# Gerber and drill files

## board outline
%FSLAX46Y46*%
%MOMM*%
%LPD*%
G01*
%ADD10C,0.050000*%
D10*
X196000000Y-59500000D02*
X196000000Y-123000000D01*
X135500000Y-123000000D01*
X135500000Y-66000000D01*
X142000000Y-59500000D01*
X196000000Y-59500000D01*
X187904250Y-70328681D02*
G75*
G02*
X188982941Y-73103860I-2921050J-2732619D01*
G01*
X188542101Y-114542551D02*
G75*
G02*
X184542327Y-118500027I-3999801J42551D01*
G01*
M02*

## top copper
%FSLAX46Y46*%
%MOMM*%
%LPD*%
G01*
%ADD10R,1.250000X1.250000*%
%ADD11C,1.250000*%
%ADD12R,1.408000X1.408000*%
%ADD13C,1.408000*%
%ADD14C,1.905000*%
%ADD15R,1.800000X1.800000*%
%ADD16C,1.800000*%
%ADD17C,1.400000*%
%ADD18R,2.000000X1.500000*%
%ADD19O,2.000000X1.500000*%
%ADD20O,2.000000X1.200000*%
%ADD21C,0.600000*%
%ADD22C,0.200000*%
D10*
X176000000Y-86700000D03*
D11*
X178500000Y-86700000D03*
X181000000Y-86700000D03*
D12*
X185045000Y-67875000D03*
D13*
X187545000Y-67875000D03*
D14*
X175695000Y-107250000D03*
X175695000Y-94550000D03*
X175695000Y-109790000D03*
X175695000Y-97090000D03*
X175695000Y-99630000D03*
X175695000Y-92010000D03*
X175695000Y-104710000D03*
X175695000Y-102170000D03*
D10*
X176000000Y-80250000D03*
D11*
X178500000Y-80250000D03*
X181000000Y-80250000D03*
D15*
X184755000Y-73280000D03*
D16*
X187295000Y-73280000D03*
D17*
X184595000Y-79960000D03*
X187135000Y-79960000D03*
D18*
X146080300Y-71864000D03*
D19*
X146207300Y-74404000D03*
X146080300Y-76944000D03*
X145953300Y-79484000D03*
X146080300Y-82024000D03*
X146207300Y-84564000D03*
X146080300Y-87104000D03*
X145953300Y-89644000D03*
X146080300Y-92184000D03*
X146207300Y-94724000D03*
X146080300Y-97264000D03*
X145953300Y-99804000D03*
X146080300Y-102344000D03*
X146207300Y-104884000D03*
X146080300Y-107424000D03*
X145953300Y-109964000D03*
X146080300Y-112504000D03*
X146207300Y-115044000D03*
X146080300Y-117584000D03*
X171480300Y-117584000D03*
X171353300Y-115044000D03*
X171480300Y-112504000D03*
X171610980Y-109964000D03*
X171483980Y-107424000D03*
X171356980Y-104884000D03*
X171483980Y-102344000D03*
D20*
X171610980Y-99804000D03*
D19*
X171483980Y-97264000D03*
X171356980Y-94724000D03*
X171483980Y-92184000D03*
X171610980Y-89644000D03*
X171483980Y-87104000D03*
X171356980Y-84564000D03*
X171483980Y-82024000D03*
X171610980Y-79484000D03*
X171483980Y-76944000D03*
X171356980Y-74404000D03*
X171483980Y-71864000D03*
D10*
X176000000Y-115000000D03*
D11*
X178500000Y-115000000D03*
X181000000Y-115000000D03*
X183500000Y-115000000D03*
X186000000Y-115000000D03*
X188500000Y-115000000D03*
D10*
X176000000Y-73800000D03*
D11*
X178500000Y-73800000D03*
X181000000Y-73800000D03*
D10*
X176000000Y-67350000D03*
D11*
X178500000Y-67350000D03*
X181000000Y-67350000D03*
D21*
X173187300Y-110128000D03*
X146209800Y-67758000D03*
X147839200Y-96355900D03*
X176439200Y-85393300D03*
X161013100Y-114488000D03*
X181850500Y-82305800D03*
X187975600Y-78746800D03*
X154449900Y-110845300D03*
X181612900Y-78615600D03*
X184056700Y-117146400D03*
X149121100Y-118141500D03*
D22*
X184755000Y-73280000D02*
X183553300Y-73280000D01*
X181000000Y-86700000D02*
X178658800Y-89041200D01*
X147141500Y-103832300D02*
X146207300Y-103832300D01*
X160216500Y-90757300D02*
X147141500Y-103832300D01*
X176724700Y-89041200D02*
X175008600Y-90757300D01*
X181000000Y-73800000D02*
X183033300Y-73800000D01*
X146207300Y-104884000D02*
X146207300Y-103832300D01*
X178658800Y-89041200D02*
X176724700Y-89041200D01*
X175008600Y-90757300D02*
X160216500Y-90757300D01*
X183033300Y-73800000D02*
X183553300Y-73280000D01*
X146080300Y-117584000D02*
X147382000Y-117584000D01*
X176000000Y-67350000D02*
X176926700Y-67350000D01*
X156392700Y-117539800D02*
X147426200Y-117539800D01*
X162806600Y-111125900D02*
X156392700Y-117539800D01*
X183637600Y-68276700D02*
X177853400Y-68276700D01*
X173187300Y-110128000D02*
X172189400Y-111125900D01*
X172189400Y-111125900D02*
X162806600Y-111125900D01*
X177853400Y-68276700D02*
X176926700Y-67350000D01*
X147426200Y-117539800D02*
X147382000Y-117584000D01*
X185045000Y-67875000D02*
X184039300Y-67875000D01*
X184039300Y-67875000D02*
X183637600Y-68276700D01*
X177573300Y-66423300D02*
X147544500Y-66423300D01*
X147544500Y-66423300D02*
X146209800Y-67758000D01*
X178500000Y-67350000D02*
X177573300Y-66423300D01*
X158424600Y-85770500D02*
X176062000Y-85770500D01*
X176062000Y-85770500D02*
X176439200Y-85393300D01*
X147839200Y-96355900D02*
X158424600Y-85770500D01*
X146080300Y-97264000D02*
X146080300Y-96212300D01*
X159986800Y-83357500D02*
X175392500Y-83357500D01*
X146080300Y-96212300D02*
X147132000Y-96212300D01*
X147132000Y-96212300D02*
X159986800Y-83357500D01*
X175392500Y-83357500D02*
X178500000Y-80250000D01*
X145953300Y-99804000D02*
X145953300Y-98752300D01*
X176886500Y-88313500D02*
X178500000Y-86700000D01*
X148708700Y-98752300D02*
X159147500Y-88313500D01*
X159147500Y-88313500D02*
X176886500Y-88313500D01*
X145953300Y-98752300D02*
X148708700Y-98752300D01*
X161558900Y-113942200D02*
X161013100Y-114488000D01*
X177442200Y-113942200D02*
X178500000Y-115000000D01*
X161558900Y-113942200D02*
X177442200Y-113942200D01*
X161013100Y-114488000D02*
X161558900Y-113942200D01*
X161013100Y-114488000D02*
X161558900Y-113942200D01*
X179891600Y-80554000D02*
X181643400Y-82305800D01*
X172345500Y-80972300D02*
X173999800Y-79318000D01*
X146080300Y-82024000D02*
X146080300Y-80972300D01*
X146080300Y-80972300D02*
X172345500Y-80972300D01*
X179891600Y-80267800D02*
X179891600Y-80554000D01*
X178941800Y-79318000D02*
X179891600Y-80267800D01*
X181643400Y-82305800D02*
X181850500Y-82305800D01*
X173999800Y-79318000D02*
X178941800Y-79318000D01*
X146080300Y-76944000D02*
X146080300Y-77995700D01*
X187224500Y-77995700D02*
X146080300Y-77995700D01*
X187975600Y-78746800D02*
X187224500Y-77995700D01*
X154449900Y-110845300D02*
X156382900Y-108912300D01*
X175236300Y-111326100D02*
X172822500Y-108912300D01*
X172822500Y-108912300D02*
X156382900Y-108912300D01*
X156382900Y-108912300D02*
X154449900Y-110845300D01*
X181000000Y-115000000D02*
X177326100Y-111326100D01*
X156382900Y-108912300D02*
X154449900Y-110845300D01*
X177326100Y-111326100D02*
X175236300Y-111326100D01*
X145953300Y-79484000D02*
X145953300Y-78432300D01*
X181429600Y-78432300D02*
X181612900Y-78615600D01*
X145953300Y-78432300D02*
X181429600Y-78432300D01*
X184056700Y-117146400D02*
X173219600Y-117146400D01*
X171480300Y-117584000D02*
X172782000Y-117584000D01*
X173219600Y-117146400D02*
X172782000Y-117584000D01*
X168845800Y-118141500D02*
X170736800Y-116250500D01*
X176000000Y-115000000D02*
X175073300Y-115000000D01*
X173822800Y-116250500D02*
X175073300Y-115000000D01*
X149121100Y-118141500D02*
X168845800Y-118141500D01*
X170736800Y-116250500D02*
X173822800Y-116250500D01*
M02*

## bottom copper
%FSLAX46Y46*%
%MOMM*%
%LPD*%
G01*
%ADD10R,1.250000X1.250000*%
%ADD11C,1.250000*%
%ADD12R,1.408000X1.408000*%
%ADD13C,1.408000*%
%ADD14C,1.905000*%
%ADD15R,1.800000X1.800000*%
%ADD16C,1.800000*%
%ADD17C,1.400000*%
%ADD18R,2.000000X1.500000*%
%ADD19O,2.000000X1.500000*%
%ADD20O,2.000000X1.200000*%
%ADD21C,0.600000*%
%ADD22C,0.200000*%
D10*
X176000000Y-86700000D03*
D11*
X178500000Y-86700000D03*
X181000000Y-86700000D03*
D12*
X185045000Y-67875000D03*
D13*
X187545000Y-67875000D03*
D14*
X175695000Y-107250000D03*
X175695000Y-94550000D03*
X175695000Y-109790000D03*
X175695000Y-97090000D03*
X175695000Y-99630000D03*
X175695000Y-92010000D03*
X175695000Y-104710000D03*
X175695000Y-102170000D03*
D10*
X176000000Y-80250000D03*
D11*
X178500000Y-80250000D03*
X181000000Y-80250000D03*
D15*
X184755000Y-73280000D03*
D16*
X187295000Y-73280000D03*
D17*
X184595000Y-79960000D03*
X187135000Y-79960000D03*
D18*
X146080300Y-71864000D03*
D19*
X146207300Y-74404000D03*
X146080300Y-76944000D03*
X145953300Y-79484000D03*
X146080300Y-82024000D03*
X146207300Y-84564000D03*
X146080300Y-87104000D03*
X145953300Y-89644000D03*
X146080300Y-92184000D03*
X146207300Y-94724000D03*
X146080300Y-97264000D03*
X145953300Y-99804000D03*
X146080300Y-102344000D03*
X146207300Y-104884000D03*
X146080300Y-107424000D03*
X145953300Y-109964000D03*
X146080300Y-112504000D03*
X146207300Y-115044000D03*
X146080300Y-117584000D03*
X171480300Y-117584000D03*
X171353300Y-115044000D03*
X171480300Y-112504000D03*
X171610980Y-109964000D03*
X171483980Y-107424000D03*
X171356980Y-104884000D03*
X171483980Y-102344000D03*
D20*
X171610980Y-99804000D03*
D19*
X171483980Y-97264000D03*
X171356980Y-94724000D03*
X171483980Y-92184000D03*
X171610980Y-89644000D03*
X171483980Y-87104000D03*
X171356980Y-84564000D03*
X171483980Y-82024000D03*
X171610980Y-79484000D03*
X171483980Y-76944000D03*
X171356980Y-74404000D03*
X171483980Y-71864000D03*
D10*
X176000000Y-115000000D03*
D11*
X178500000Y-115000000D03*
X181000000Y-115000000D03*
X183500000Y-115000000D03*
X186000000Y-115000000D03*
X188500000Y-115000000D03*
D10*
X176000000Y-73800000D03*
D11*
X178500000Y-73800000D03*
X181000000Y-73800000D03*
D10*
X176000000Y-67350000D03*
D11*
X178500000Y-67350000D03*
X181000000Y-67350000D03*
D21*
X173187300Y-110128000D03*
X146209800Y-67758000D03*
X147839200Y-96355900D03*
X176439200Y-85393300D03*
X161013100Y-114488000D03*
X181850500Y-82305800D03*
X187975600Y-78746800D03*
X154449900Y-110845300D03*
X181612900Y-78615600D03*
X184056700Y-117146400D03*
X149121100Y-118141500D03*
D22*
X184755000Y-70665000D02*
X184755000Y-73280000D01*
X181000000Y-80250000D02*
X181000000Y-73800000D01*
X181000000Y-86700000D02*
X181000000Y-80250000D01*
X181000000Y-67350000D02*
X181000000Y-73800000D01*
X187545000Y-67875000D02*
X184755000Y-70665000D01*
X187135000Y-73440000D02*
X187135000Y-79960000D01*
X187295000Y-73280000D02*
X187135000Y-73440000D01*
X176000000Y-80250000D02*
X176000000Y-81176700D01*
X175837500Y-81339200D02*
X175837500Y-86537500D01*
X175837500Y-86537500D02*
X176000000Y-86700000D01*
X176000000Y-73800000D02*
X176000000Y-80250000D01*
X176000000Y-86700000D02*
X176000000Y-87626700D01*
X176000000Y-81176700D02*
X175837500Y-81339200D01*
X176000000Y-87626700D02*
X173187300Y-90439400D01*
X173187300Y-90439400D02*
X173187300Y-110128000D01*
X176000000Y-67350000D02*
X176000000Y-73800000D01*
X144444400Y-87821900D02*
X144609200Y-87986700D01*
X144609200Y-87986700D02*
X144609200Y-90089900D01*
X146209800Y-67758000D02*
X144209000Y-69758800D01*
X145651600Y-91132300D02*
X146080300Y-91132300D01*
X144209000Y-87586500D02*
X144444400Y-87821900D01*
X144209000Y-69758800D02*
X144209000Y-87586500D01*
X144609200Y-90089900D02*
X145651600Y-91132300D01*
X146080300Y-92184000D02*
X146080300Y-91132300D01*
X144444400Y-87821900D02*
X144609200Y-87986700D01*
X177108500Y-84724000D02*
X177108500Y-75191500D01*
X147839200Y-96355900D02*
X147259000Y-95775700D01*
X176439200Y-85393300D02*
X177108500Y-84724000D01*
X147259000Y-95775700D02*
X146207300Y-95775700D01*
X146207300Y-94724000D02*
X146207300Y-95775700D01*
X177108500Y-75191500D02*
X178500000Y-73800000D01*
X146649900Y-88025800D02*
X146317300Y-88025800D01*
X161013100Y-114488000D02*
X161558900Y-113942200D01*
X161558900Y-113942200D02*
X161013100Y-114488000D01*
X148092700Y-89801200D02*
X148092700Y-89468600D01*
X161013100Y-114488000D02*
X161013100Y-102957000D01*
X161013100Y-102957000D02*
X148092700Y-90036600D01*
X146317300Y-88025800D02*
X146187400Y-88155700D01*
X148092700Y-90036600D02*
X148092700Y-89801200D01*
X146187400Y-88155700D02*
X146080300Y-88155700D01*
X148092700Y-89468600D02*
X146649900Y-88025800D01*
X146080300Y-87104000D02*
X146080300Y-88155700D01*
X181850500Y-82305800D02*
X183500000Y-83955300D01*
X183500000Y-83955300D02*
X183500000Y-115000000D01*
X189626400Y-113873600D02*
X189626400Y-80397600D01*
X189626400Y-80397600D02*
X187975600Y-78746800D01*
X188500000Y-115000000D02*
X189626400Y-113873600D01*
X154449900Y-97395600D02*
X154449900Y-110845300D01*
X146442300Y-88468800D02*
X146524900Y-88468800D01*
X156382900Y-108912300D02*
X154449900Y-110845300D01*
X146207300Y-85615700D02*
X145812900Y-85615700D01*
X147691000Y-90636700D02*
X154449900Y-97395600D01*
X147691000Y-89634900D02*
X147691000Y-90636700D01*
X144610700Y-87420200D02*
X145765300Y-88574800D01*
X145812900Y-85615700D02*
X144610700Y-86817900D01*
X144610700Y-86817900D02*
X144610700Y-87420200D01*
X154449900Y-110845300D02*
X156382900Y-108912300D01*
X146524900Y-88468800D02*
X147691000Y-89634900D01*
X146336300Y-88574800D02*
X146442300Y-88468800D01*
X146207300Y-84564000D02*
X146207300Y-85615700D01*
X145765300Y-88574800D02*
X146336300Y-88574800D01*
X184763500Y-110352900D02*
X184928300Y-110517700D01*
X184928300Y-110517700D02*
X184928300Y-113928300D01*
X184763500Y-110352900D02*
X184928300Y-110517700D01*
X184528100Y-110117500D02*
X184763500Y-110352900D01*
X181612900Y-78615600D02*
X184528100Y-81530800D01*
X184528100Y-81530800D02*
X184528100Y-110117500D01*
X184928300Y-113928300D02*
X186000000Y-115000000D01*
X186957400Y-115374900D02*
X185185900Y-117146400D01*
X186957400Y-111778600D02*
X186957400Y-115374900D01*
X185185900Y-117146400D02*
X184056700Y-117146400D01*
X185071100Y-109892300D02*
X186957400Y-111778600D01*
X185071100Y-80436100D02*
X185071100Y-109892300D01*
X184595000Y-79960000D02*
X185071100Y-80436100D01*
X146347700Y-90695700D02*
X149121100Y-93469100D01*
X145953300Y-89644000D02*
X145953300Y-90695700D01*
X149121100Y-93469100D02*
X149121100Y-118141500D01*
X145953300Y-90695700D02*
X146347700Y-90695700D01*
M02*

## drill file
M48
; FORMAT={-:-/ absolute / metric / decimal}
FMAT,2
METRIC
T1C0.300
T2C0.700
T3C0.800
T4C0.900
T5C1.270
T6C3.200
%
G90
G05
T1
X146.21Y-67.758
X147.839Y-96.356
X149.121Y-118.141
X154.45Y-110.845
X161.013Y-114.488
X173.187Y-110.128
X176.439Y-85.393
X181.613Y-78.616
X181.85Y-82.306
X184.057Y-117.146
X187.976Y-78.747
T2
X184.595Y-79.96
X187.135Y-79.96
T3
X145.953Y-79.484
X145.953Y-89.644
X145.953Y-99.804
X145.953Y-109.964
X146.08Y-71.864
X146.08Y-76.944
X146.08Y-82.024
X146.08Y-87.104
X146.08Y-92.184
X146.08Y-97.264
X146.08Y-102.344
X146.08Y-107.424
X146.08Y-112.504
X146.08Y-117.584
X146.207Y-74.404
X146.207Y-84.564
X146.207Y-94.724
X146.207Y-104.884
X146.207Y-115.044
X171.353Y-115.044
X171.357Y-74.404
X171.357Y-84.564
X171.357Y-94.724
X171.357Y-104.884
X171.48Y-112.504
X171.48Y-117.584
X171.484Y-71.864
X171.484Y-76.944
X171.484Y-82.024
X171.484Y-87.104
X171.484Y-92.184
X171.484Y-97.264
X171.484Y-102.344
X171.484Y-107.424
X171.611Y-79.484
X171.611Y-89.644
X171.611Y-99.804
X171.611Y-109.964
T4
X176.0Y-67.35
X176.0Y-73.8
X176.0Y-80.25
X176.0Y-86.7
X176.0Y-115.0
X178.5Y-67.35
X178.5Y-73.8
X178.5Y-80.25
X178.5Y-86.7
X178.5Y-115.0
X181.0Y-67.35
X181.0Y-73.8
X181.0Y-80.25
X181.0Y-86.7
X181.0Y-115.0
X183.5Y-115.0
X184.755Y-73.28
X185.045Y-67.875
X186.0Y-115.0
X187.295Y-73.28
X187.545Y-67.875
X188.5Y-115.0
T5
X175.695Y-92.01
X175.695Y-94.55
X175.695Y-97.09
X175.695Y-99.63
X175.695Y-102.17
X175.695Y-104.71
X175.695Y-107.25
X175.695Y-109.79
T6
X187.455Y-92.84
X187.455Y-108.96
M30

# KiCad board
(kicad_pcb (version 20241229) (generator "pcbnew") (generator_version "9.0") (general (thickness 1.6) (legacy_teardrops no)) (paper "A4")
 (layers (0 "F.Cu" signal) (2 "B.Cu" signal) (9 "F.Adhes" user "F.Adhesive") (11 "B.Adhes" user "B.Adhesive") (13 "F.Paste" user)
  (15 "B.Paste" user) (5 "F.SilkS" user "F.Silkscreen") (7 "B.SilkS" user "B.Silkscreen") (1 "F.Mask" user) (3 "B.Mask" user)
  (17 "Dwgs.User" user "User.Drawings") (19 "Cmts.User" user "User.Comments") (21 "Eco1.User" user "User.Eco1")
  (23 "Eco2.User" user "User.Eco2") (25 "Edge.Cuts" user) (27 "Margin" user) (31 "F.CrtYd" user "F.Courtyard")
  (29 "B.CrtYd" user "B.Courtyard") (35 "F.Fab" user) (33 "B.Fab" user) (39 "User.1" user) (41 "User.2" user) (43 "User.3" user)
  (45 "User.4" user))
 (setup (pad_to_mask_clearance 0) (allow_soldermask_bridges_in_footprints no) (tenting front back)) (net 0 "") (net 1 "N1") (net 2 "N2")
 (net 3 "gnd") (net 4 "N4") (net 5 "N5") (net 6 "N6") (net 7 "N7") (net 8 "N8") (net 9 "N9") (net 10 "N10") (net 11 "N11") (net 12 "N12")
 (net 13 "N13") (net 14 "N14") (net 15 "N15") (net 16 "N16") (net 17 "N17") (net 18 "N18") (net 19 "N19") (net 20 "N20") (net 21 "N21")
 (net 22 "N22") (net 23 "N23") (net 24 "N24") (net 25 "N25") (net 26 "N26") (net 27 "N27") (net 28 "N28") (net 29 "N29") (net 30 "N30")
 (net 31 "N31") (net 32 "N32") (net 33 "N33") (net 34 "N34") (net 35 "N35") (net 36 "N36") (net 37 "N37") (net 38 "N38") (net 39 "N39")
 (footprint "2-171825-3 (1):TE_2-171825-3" (layer "F.Cu") (at 176 86.7)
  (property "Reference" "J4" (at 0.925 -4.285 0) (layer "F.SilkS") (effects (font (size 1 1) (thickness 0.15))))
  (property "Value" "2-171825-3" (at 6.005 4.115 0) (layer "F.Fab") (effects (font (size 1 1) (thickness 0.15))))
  (pad "1" thru_hole rect (at 0 0) (size 1.25 1.25) (drill 0.9) (layers "*.Cu" "*.Mask") (remove_unused_layers no) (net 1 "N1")
   (solder_mask_margin 0.102))
  (pad "2" thru_hole circle (at 2.5 0) (size 1.25 1.25) (drill 0.9) (layers "*.Cu" "*.Mask") (remove_unused_layers no) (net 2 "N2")
   (solder_mask_margin 0.102))
  (pad "3" thru_hole circle (at 5 0) (size 1.25 1.25) (drill 0.9) (layers "*.Cu" "*.Mask") (remove_unused_layers no) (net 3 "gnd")
   (solder_mask_margin 0.102)))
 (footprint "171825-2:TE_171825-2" (layer "F.Cu") (at 186.295 67.875)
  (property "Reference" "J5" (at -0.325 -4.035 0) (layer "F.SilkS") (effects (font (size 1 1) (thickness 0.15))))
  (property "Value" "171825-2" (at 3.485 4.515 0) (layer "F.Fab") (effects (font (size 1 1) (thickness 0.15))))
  (pad "1" thru_hole rect (at -1.25 0) (size 1.408 1.408) (drill 0.9) (layers "*.Cu" "*.Mask") (remove_unused_layers no) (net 1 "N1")
   (solder_mask_margin 0.102))
  (pad "2" thru_hole circle (at 1.25 0) (size 1.408 1.408) (drill 0.9) (layers "*.Cu" "*.Mask") (remove_unused_layers no) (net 3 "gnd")
   (solder_mask_margin 0.102)))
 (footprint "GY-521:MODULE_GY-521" (layer "F.Cu") (at 182.025 100.9)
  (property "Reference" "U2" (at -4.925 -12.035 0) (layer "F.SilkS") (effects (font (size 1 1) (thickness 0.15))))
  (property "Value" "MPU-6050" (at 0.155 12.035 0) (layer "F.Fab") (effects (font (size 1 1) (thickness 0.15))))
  (pad "" np_thru_hole circle (at 5.43 -8.06) (size 3.2 3.2) (drill 3.2) (layers "*.Cu" "*.Mask"))
  (pad "" np_thru_hole circle (at 5.43 8.06) (size 3.2 3.2) (drill 3.2) (layers "*.Cu" "*.Mask"))
  (pad "AD0" thru_hole circle (at -6.33 6.35) (size 1.905 1.905) (drill 1.27) (layers "*.Cu" "*.Mask") (remove_unused_layers no)
   (solder_mask_margin 0.102))
  (pad "GND" thru_hole circle (at -6.33 -6.35) (size 1.905 1.905) (drill 1.27) (layers "*.Cu" "*.Mask") (remove_unused_layers no)
   (solder_mask_margin 0.102))
  (pad "INT" thru_hole circle (at -6.33 8.89) (size 1.905 1.905) (drill 1.27) (layers "*.Cu" "*.Mask") (remove_unused_layers no)
   (solder_mask_margin 0.102))
  (pad "SCL" thru_hole circle (at -6.33 -3.81) (size 1.905 1.905) (drill 1.27) (layers "*.Cu" "*.Mask") (remove_unused_layers no)
   (solder_mask_margin 0.102))
  (pad "SDA" thru_hole circle (at -6.33 -1.27) (size 1.905 1.905) (drill 1.27) (layers "*.Cu" "*.Mask") (remove_unused_layers no)
   (solder_mask_margin 0.102))
  (pad "VCC" thru_hole circle (at -6.33 -8.89) (size 1.905 1.905) (drill 1.27) (layers "*.Cu" "*.Mask") (remove_unused_layers no)
   (solder_mask_margin 0.102))
  (pad "XCL" thru_hole circle (at -6.33 3.81) (size 1.905 1.905) (drill 1.27) (layers "*.Cu" "*.Mask") (remove_unused_layers no)
   (solder_mask_margin 0.102))
  (pad "XDA" thru_hole circle (at -6.33 1.27) (size 1.905 1.905) (drill 1.27) (layers "*.Cu" "*.Mask") (remove_unused_layers no)
   (solder_mask_margin 0.102)))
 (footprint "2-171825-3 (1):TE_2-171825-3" (layer "F.Cu") (at 176 80.25)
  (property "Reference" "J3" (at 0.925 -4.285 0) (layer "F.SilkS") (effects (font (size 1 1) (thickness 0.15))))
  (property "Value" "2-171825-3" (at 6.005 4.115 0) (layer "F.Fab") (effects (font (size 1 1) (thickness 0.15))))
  (pad "1" thru_hole rect (at 0 0) (size 1.25 1.25) (drill 0.9) (layers "*.Cu" "*.Mask") (remove_unused_layers no) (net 1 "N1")
   (solder_mask_margin 0.102))
  (pad "2" thru_hole circle (at 2.5 0) (size 1.25 1.25) (drill 0.9) (layers "*.Cu" "*.Mask") (remove_unused_layers no) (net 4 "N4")
   (solder_mask_margin 0.102))
  (pad "3" thru_hole circle (at 5 0) (size 1.25 1.25) (drill 0.9) (layers "*.Cu" "*.Mask") (remove_unused_layers no) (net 3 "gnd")
   (solder_mask_margin 0.102)))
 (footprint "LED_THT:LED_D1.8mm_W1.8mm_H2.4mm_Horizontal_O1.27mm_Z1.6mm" (layer "F.Cu") (at 184.755 73.28)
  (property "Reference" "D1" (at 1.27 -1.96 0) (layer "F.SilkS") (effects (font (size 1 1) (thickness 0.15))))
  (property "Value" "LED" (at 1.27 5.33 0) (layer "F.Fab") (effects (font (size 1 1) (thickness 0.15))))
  (pad "1" thru_hole rect (at 0 0) (size 1.8 1.8) (drill 0.9) (layers "*.Cu" "*.Mask") (remove_unused_layers no) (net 3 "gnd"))
  (pad "2" thru_hole circle (at 2.54 0) (size 1.8 1.8) (drill 0.9) (layers "*.Cu" "*.Mask") (remove_unused_layers no) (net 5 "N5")))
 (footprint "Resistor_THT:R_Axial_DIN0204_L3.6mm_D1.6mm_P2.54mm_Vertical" (layer "F.Cu") (at 184.595 79.96)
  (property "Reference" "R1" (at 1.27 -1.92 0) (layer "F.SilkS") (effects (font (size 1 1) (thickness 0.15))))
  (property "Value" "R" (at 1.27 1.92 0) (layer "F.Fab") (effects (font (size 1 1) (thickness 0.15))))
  (pad "1" thru_hole circle (at 0 0) (size 1.4 1.4) (drill 0.7) (layers "*.Cu" "*.Mask") (remove_unused_layers no) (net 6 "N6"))
  (pad "2" thru_hole circle (at 2.54 0) (size 1.4 1.4) (drill 0.7) (layers "*.Cu" "*.Mask") (remove_unused_layers no) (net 5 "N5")))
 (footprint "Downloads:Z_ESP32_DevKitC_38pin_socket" (layer "F.Cu") (at 146.0803 71.864)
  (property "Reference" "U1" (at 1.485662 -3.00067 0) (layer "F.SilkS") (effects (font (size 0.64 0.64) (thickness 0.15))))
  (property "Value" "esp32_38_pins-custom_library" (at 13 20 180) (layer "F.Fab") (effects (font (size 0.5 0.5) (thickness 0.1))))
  (pad "1" thru_hole rect (at 0 0 270) (size 1.5 2) (drill 0.8) (layers "*.Cu" "*.Mask") (remove_unused_layers no) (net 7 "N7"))
  (pad "2" thru_hole oval (at 0.127 2.54 270) (size 1.5 2) (drill 0.8) (layers "*.Cu" "*.Mask") (remove_unused_layers no) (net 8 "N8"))
  (pad "3" thru_hole oval (at 0 5.08 270) (size 1.5 2) (drill 0.8) (layers "*.Cu" "*.Mask") (remove_unused_layers no) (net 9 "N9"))
  (pad "4" thru_hole oval (at -0.127 7.62 270) (size 1.5 2) (drill 0.8) (layers "*.Cu" "*.Mask") (remove_unused_layers no) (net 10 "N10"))
  (pad "5" thru_hole oval (at 0 10.16 270) (size 1.5 2) (drill 0.8) (layers "*.Cu" "*.Mask") (remove_unused_layers no) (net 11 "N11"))
  (pad "6" thru_hole oval (at 0.127 12.7 270) (size 1.5 2) (drill 0.8) (layers "*.Cu" "*.Mask") (remove_unused_layers no) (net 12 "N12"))
  (pad "7" thru_hole oval (at 0 15.24 270) (size 1.5 2) (drill 0.8) (layers "*.Cu" "*.Mask") (remove_unused_layers no) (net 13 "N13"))
  (pad "8" thru_hole oval (at -0.127 17.78 270) (size 1.5 2) (drill 0.8) (layers "*.Cu" "*.Mask") (remove_unused_layers no) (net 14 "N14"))
  (pad "9" thru_hole oval (at 0 20.32 270) (size 1.5 2) (drill 0.8) (layers "*.Cu" "*.Mask") (remove_unused_layers no) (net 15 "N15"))
  (pad "10" thru_hole oval (at 0.127 22.86 270) (size 1.5 2) (drill 0.8) (layers "*.Cu" "*.Mask") (remove_unused_layers no) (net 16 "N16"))
  (pad "11" thru_hole oval (at 0 25.4 270) (size 1.5 2) (drill 0.8) (layers "*.Cu" "*.Mask") (remove_unused_layers no) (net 4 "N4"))
  (pad "12" thru_hole oval (at -0.127 27.94 270) (size 1.5 2) (drill 0.8) (layers "*.Cu" "*.Mask") (remove_unused_layers no) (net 2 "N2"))
  (pad "13" thru_hole oval (at 0 30.48 270) (size 1.5 2) (drill 0.8) (layers "*.Cu" "*.Mask") (remove_unused_layers no) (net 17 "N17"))
  (pad "14" thru_hole oval (at 0.127 33.02 270) (size 1.5 2) (drill 0.8) (layers "*.Cu" "*.Mask") (remove_unused_layers no) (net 3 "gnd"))
  (pad "15" thru_hole oval (at 0 35.56 270) (size 1.5 2) (drill 0.8) (layers "*.Cu" "*.Mask") (remove_unused_layers no) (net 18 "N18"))
  (pad "16" thru_hole oval (at -0.127 38.1 270) (size 1.5 2) (drill 0.8) (layers "*.Cu" "*.Mask") (remove_unused_layers no) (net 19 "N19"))
  (pad "17" thru_hole oval (at 0 40.64 270) (size 1.5 2) (drill 0.8) (layers "*.Cu" "*.Mask") (remove_unused_layers no) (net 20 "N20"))
  (pad "18" thru_hole oval (at 0.127 43.18 270) (size 1.5 2) (drill 0.8) (layers "*.Cu" "*.Mask") (remove_unused_layers no) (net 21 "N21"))
  (pad "19" thru_hole oval (at 0 45.72 270) (size 1.5 2) (drill 0.8) (layers "*.Cu" "*.Mask") (remove_unused_layers no) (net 1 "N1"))
  (pad "20" thru_hole oval (at 25.4 45.72 270) (size 1.5 2) (drill 0.8) (layers "*.Cu" "*.Mask") (remove_unused_layers no) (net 6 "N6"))
  (pad "21" thru_hole oval (at 25.273 43.18 270) (size 1.5 2) (drill 0.8) (layers "*.Cu" "*.Mask") (remove_unused_layers no) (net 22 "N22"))
  (pad "22" thru_hole oval (at 25.4 40.64 270) (size 1.5 2) (drill 0.8) (layers "*.Cu" "*.Mask") (remove_unused_layers no) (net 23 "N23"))
  (pad "23" thru_hole oval (at 25.53068 38.1 270) (size 1.5 2) (drill 0.8) (layers "*.Cu" "*.Mask") (remove_unused_layers no) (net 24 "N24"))
  (pad "24" thru_hole oval (at 25.40368 35.56 270) (size 1.5 2) (drill 0.8) (layers "*.Cu" "*.Mask") (remove_unused_layers no)
   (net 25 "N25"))
  (pad "25" thru_hole oval (at 25.27668 33.02 270) (size 1.5 2) (drill 0.8) (layers "*.Cu" "*.Mask") (remove_unused_layers no)
   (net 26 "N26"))
  (pad "26" thru_hole oval (at 25.40368 30.48 270) (size 1.5 2) (drill 0.8) (layers "*.Cu" "*.Mask") (remove_unused_layers no)
   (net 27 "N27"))
  (pad "27" thru_hole oval (at 25.53068 27.94 270) (size 1.2 2) (drill 0.8) (layers "*.Cu" "*.Mask") (remove_unused_layers no)
   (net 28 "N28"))
  (pad "28" thru_hole oval (at 25.40368 25.4 270) (size 1.5 2) (drill 0.8) (layers "*.Cu" "*.Mask") (remove_unused_layers no) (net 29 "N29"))
  (pad "29" thru_hole oval (at 25.27668 22.86 270) (size 1.5 2) (drill 0.8) (layers "*.Cu" "*.Mask") (remove_unused_layers no)
   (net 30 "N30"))
  (pad "30" thru_hole oval (at 25.40368 20.32 270) (size 1.5 2) (drill 0.8) (layers "*.Cu" "*.Mask") (remove_unused_layers no)
   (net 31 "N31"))
  (pad "31" thru_hole oval (at 25.53068 17.78 270) (size 1.5 2) (drill 0.8) (layers "*.Cu" "*.Mask") (remove_unused_layers no)
   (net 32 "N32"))
  (pad "32" thru_hole oval (at 25.40368 15.24 270) (size 1.5 2) (drill 0.8) (layers "*.Cu" "*.Mask") (remove_unused_layers no)
   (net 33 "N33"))
  (pad "33" thru_hole oval (at 25.27668 12.7 270) (size 1.5 2) (drill 0.8) (layers "*.Cu" "*.Mask") (remove_unused_layers no) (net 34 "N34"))
  (pad "34" thru_hole oval (at 25.40368 10.16 270) (size 1.5 2) (drill 0.8) (layers "*.Cu" "*.Mask") (remove_unused_layers no)
   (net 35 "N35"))
  (pad "35" thru_hole oval (at 25.53068 7.62 270) (size 1.5 2) (drill 0.8) (layers "*.Cu" "*.Mask") (remove_unused_layers no) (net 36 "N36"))
  (pad "36" thru_hole oval (at 25.40368 5.08 270) (size 1.5 2) (drill 0.8) (layers "*.Cu" "*.Mask") (remove_unused_layers no) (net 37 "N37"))
  (pad "37" thru_hole oval (at 25.27668 2.54 270) (size 1.5 2) (drill 0.8) (layers "*.Cu" "*.Mask") (remove_unused_layers no) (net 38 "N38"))
  (pad "38" thru_hole oval (at 25.40368 0 270) (size 1.5 2) (drill 0.8) (layers "*.Cu" "*.Mask") (remove_unused_layers no) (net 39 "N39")))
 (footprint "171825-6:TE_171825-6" (layer "F.Cu") (at 176 115)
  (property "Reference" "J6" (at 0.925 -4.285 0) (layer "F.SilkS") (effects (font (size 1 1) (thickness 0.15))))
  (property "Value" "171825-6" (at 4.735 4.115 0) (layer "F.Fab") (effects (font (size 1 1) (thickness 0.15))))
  (pad "1" thru_hole rect (at 0 0) (size 1.25 1.25) (drill 0.9) (layers "*.Cu" "*.Mask") (remove_unused_layers no) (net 14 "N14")
   (solder_mask_margin 0.102))
  (pad "2" thru_hole circle (at 2.5 0) (size 1.25 1.25) (drill 0.9) (layers "*.Cu" "*.Mask") (remove_unused_layers no) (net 13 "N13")
   (solder_mask_margin 0.102))
  (pad "3" thru_hole circle (at 5 0) (size 1.25 1.25) (drill 0.9) (layers "*.Cu" "*.Mask") (remove_unused_layers no) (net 12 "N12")
   (solder_mask_margin 0.102))
  (pad "4" thru_hole circle (at 7.5 0) (size 1.25 1.25) (drill 0.9) (layers "*.Cu" "*.Mask") (remove_unused_layers no) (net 11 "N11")
   (solder_mask_margin 0.102))
  (pad "5" thru_hole circle (at 10 0) (size 1.25 1.25) (drill 0.9) (layers "*.Cu" "*.Mask") (remove_unused_layers no) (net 10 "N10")
   (solder_mask_margin 0.102))
  (pad "6" thru_hole circle (at 12.5 0) (size 1.25 1.25) (drill 0.9) (layers "*.Cu" "*.Mask") (remove_unused_layers no) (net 9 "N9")
   (solder_mask_margin 0.102)))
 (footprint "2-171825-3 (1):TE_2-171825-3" (layer "F.Cu") (at 176 73.8)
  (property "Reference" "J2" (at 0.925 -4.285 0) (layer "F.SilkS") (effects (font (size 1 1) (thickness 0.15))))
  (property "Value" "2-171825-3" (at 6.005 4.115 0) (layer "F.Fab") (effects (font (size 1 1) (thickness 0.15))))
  (pad "1" thru_hole rect (at 0 0) (size 1.25 1.25) (drill 0.9) (layers "*.Cu" "*.Mask") (remove_unused_layers no) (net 1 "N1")
   (solder_mask_margin 0.102))
  (pad "2" thru_hole circle (at 2.5 0) (size 1.25 1.25) (drill 0.9) (layers "*.Cu" "*.Mask") (remove_unused_layers no) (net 16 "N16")
   (solder_mask_margin 0.102))
  (pad "3" thru_hole circle (at 5 0) (size 1.25 1.25) (drill 0.9) (layers "*.Cu" "*.Mask") (remove_unused_layers no) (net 3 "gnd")
   (solder_mask_margin 0.102)))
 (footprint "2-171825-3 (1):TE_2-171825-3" (layer "F.Cu") (at 176 67.35)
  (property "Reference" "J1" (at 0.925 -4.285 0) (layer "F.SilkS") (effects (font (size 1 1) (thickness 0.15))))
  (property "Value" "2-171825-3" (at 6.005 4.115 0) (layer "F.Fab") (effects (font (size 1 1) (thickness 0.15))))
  (pad "1" thru_hole rect (at 0 0) (size 1.25 1.25) (drill 0.9) (layers "*.Cu" "*.Mask") (remove_unused_layers no) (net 1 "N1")
   (solder_mask_margin 0.102))
  (pad "2" thru_hole circle (at 2.5 0) (size 1.25 1.25) (drill 0.9) (layers "*.Cu" "*.Mask") (remove_unused_layers no) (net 15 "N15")
   (solder_mask_margin 0.102))
  (pad "3" thru_hole circle (at 5 0) (size 1.25 1.25) (drill 0.9) (layers "*.Cu" "*.Mask") (remove_unused_layers no) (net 3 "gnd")
   (solder_mask_margin 0.102)))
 (gr_poly
  (pts (xy 196 59.5) (xy 196 123) (xy 135.5 123) (xy 135.5 66) (xy 142 59.5)) (stroke (width 0.05) (type solid)) (fill no)
  (layer "Edge.Cuts"))
 (gr_arc (start 187.90425 70.328681) (mid 188.711432 71.612164) (end 188.982938 73.10386) (stroke (width 0.05) (type default))
  (layer "Edge.Cuts"))
 (gr_arc (start 188.542101 114.542551) (mid 187.35567 117.343432) (end 184.542327 118.5) (stroke (width 0.05) (type default))
  (layer "Edge.Cuts"))
 (segment (start 184.755 73.28) (end 183.5533 73.28) (width 0.2) (layer "F.Cu") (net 3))
 (segment (start 181 86.7) (end 178.6588 89.0412) (width 0.2) (layer "F.Cu") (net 3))
 (segment (start 147.1415 103.8323) (end 146.2073 103.8323) (width 0.2) (layer "F.Cu") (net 3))
 (segment (start 160.2165 90.7573) (end 147.1415 103.8323) (width 0.2) (layer "F.Cu") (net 3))
 (segment (start 176.7247 89.0412) (end 175.0086 90.7573) (width 0.2) (layer "F.Cu") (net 3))
 (segment (start 181 73.8) (end 183.0333 73.8) (width 0.2) (layer "F.Cu") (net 3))
 (segment (start 146.2073 104.884) (end 146.2073 103.8323) (width 0.2) (layer "F.Cu") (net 3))
 (segment (start 178.6588 89.0412) (end 176.7247 89.0412) (width 0.2) (layer "F.Cu") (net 3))
 (segment (start 175.0086 90.7573) (end 160.2165 90.7573) (width 0.2) (layer "F.Cu") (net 3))
 (segment (start 183.0333 73.8) (end 183.5533 73.28) (width 0.2) (layer "F.Cu") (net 3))
 (segment (start 184.755 70.665) (end 184.755 73.28) (width 0.2) (layer "B.Cu") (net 3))
 (segment (start 181 80.25) (end 181 73.8) (width 0.2) (layer "B.Cu") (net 3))
 (segment (start 181 86.7) (end 181 80.25) (width 0.2) (layer "B.Cu") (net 3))
 (segment (start 181 67.35) (end 181 73.8) (width 0.2) (layer "B.Cu") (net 3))
 (segment (start 187.545 67.875) (end 184.755 70.665) (width 0.2) (layer "B.Cu") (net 3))
 (segment (start 187.135 73.44) (end 187.135 79.96) (width 0.2) (layer "B.Cu") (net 5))
 (segment (start 187.295 73.28) (end 187.135 73.44) (width 0.2) (layer "B.Cu") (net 5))
 (segment (start 146.0803 117.584) (end 147.382 117.584) (width 0.2) (layer "F.Cu") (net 1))
 (segment (start 176 67.35) (end 176.9267 67.35) (width 0.2) (layer "F.Cu") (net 1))
 (segment (start 156.3927 117.5398) (end 147.4262 117.5398) (width 0.2) (layer "F.Cu") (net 1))
 (segment (start 162.8066 111.1259) (end 156.3927 117.5398) (width 0.2) (layer "F.Cu") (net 1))
 (segment (start 183.6376 68.2767) (end 177.8534 68.2767) (width 0.2) (layer "F.Cu") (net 1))
 (segment (start 173.1873 110.128) (end 172.1894 111.1259) (width 0.2) (layer "F.Cu") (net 1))
 (segment (start 172.1894 111.1259) (end 162.8066 111.1259) (width 0.2) (layer "F.Cu") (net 1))
 (segment (start 177.8534 68.2767) (end 176.9267 67.35) (width 0.2) (layer "F.Cu") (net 1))
 (segment (start 147.4262 117.5398) (end 147.382 117.584) (width 0.2) (layer "F.Cu") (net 1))
 (segment (start 185.045 67.875) (end 184.0393 67.875) (width 0.2) (layer "F.Cu") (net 1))
 (segment (start 184.0393 67.875) (end 183.6376 68.2767) (width 0.2) (layer "F.Cu") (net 1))
 (via (at 173.1873 110.128) (size 0.6) (drill 0.3) (layers "F.Cu" "B.Cu") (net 1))
 (segment (start 176 80.25) (end 176 81.1767) (width 0.2) (layer "B.Cu") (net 1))
 (segment (start 175.8375 81.3392) (end 175.8375 86.5375) (width 0.2) (layer "B.Cu") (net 1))
 (segment (start 175.8375 86.5375) (end 176 86.7) (width 0.2) (layer "B.Cu") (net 1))
 (segment (start 176 73.8) (end 176 80.25) (width 0.2) (layer "B.Cu") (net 1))
 (segment (start 176 86.7) (end 176 87.6267) (width 0.2) (layer "B.Cu") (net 1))
 (segment (start 176 81.1767) (end 175.8375 81.3392) (width 0.2) (layer "B.Cu") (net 1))
 (segment (start 176 87.6267) (end 173.1873 90.4394) (width 0.2) (layer "B.Cu") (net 1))
 (segment (start 173.1873 90.4394) (end 173.1873 110.128) (width 0.2) (layer "B.Cu") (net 1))
 (segment (start 176 67.35) (end 176 73.8) (width 0.2) (layer "B.Cu") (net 1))
 (segment (start 177.5733 66.4233) (end 147.5445 66.4233) (width 0.2) (layer "F.Cu") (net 15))
 (segment (start 147.5445 66.4233) (end 146.2098 67.758) (width 0.2) (layer "F.Cu") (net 15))
 (segment (start 178.5 67.35) (end 177.5733 66.4233) (width 0.2) (layer "F.Cu") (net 15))
 (via (at 146.2098 67.758) (size 0.6) (drill 0.3) (layers "F.Cu" "B.Cu") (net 15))
 (segment (start 144.4444 87.8219) (end 144.6092 87.9867) (width 0.2) (layer "B.Cu") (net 15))
 (segment (start 144.6092 87.9867) (end 144.6092 90.0899) (width 0.2) (layer "B.Cu") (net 15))
 (segment (start 146.2098 67.758) (end 144.209 69.7588) (width 0.2) (layer "B.Cu") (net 15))
 (segment (start 145.6516 91.1323) (end 146.0803 91.1323) (width 0.2) (layer "B.Cu") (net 15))
 (segment (start 144.209 87.5865) (end 144.4444 87.8219) (width 0.2) (layer "B.Cu") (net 15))
 (segment (start 144.209 69.7588) (end 144.209 87.5865) (width 0.2) (layer "B.Cu") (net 15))
 (segment (start 144.6092 90.0899) (end 145.6516 91.1323) (width 0.2) (layer "B.Cu") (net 15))
 (segment (start 146.0803 92.184) (end 146.0803 91.1323) (width 0.2) (layer "B.Cu") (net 15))
 (segment (start 144.4444 87.8219) (end 144.6092 87.9867) (width 0.2) (layer "B.Cu") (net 15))
 (segment (start 158.4246 85.7705) (end 176.062 85.7705) (width 0.2) (layer "F.Cu") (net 16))
 (segment (start 176.062 85.7705) (end 176.4392 85.3933) (width 0.2) (layer "F.Cu") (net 16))
 (segment (start 147.8392 96.3559) (end 158.4246 85.7705) (width 0.2) (layer "F.Cu") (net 16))
 (via (at 147.8392 96.3559) (size 0.6) (drill 0.3) (layers "F.Cu" "B.Cu") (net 16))
 (via (at 176.4392 85.3933) (size 0.6) (drill 0.3) (layers "F.Cu" "B.Cu") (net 16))
 (segment (start 177.1085 84.724) (end 177.1085 75.1915) (width 0.2) (layer "B.Cu") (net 16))
 (segment (start 147.8392 96.3559) (end 147.259 95.7757) (width 0.2) (layer "B.Cu") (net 16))
 (segment (start 176.4392 85.3933) (end 177.1085 84.724) (width 0.2) (layer "B.Cu") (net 16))
 (segment (start 147.259 95.7757) (end 146.2073 95.7757) (width 0.2) (layer "B.Cu") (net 16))
 (segment (start 146.2073 94.724) (end 146.2073 95.7757) (width 0.2) (layer "B.Cu") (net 16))
 (segment (start 177.1085 75.1915) (end 178.5 73.8) (width 0.2) (layer "B.Cu") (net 16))
 (segment (start 146.0803 97.264) (end 146.0803 96.2123) (width 0.2) (layer "F.Cu") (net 4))
 (segment (start 159.9868 83.3575) (end 175.3925 83.3575) (width 0.2) (layer "F.Cu") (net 4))
 (segment (start 146.0803 96.2123) (end 147.132 96.2123) (width 0.2) (layer "F.Cu") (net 4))
 (segment (start 147.132 96.2123) (end 159.9868 83.3575) (width 0.2) (layer "F.Cu") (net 4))
 (segment (start 175.3925 83.3575) (end 178.5 80.25) (width 0.2) (layer "F.Cu") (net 4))
 (segment (start 145.9533 99.804) (end 145.9533 98.7523) (width 0.2) (layer "F.Cu") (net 2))
 (segment (start 176.8865 88.3135) (end 178.5 86.7) (width 0.2) (layer "F.Cu") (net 2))
 (segment (start 148.7087 98.7523) (end 159.1475 88.3135) (width 0.2) (layer "F.Cu") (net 2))
 (segment (start 159.1475 88.3135) (end 176.8865 88.3135) (width 0.2) (layer "F.Cu") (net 2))
 (segment (start 145.9533 98.7523) (end 148.7087 98.7523) (width 0.2) (layer "F.Cu") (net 2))
 (segment (start 161.5589 113.9422) (end 161.0131 114.488) (width 0.2) (layer "F.Cu") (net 13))
 (segment (start 177.4422 113.9422) (end 178.5 115) (width 0.2) (layer "F.Cu") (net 13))
 (segment (start 161.5589 113.9422) (end 177.4422 113.9422) (width 0.2) (layer "F.Cu") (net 13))
 (segment (start 161.0131 114.488) (end 161.5589 113.9422) (width 0.2) (layer "F.Cu") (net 13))
 (segment (start 161.0131 114.488) (end 161.5589 113.9422) (width 0.2) (layer "F.Cu") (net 13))
 (via (at 161.0131 114.488) (size 0.6) (drill 0.3) (layers "F.Cu" "B.Cu") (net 13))
 (segment (start 146.6499 88.0258) (end 146.3173 88.0258) (width 0.2) (layer "B.Cu") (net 13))
 (segment (start 161.0131 114.488) (end 161.5589 113.9422) (width 0.2) (layer "B.Cu") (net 13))
 (segment (start 161.5589 113.9422) (end 161.0131 114.488) (width 0.2) (layer "B.Cu") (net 13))
 (segment (start 148.0927 89.8012) (end 148.0927 89.4686) (width 0.2) (layer "B.Cu") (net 13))
 (segment (start 161.0131 114.488) (end 161.0131 102.957) (width 0.2) (layer "B.Cu") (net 13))
 (segment (start 161.0131 102.957) (end 148.0927 90.0366) (width 0.2) (layer "B.Cu") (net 13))
 (segment (start 146.3173 88.0258) (end 146.1874 88.1557) (width 0.2) (layer "B.Cu") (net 13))
 (segment (start 148.0927 90.0366) (end 148.0927 89.8012) (width 0.2) (layer "B.Cu") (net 13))
 (segment (start 146.1874 88.1557) (end 146.0803 88.1557) (width 0.2) (layer "B.Cu") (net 13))
 (segment (start 148.0927 89.4686) (end 146.6499 88.0258) (width 0.2) (layer "B.Cu") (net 13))
 (segment (start 146.0803 87.104) (end 146.0803 88.1557) (width 0.2) (layer "B.Cu") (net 13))
 (segment (start 179.8916 80.554) (end 181.6434 82.3058) (width 0.2) (layer "F.Cu") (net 11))
 (segment (start 172.3455 80.9723) (end 173.9998 79.318) (width 0.2) (layer "F.Cu") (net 11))
 (segment (start 146.0803 82.024) (end 146.0803 80.9723) (width 0.2) (layer "F.Cu") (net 11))
 (segment (start 146.0803 80.9723) (end 172.3455 80.9723) (width 0.2) (layer "F.Cu") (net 11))
 (segment (start 179.8916 80.2678) (end 179.8916 80.554) (width 0.2) (layer "F.Cu") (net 11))
 (segment (start 178.9418 79.318) (end 179.8916 80.2678) (width 0.2) (layer "F.Cu") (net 11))
 (segment (start 181.6434 82.3058) (end 181.8505 82.3058) (width 0.2) (layer "F.Cu") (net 11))
 (segment (start 173.9998 79.318) (end 178.9418 79.318) (width 0.2) (layer "F.Cu") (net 11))
 (via (at 181.8505 82.3058) (size 0.6) (drill 0.3) (layers "F.Cu" "B.Cu") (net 11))
 (segment (start 181.8505 82.3058) (end 183.5 83.9553) (width 0.2) (layer "B.Cu") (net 11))
 (segment (start 183.5 83.9553) (end 183.5 115) (width 0.2) (layer "B.Cu") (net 11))
 (segment (start 146.0803 76.944) (end 146.0803 77.9957) (width 0.2) (layer "F.Cu") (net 9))
 (segment (start 187.2245 77.9957) (end 146.0803 77.9957) (width 0.2) (layer "F.Cu") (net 9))
 (segment (start 187.9756 78.7468) (end 187.2245 77.9957) (width 0.2) (layer "F.Cu") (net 9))
 (via (at 187.9756 78.7468) (size 0.6) (drill 0.3) (layers "F.Cu" "B.Cu") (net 9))
 (segment (start 189.6264 113.8736) (end 189.6264 80.3976) (width 0.2) (layer "B.Cu") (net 9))
 (segment (start 189.6264 80.3976) (end 187.9756 78.7468) (width 0.2) (layer "B.Cu") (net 9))
 (segment (start 188.5 115) (end 189.6264 113.8736) (width 0.2) (layer "B.Cu") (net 9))
 (segment (start 154.4499 110.8453) (end 156.3829 108.9123) (width 0.2) (layer "F.Cu") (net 12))
 (segment (start 175.2363 111.3261) (end 172.8225 108.9123) (width 0.2) (layer "F.Cu") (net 12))
 (segment (start 172.8225 108.9123) (end 156.3829 108.9123) (width 0.2) (layer "F.Cu") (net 12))
 (segment (start 156.3829 108.9123) (end 154.4499 110.8453) (width 0.2) (layer "F.Cu") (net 12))
 (segment (start 181 115) (end 177.3261 111.3261) (width 0.2) (layer "F.Cu") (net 12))
 (segment (start 156.3829 108.9123) (end 154.4499 110.8453) (width 0.2) (layer "F.Cu") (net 12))
 (segment (start 177.3261 111.3261) (end 175.2363 111.3261) (width 0.2) (layer "F.Cu") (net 12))
 (via (at 154.4499 110.8453) (size 0.6) (drill 0.3) (layers "F.Cu" "B.Cu") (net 12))
 (segment (start 154.4499 97.3956) (end 154.4499 110.8453) (width 0.2) (layer "B.Cu") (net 12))
 (segment (start 146.4423 88.4688) (end 146.5249 88.4688) (width 0.2) (layer "B.Cu") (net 12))
 (segment (start 156.3829 108.9123) (end 154.4499 110.8453) (width 0.2) (layer "B.Cu") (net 12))
 (segment (start 146.2073 85.6157) (end 145.8129 85.6157) (width 0.2) (layer "B.Cu") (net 12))
 (segment (start 147.691 90.6367) (end 154.4499 97.3956) (width 0.2) (layer "B.Cu") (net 12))
 (segment (start 147.691 89.6349) (end 147.691 90.6367) (width 0.2) (layer "B.Cu") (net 12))
 (segment (start 144.6107 87.4202) (end 145.7653 88.5748) (width 0.2) (layer "B.Cu") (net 12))
 (segment (start 145.8129 85.6157) (end 144.6107 86.8179) (width 0.2) (layer "B.Cu") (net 12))
 (segment (start 144.6107 86.8179) (end 144.6107 87.4202) (width 0.2) (layer "B.Cu") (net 12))
 (segment (start 154.4499 110.8453) (end 156.3829 108.9123) (width 0.2) (layer "B.Cu") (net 12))
 (segment (start 146.5249 88.4688) (end 147.691 89.6349) (width 0.2) (layer "B.Cu") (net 12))
 (segment (start 146.3363 88.5748) (end 146.4423 88.4688) (width 0.2) (layer "B.Cu") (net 12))
 (segment (start 146.2073 84.564) (end 146.2073 85.6157) (width 0.2) (layer "B.Cu") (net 12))
 (segment (start 145.7653 88.5748) (end 146.3363 88.5748) (width 0.2) (layer "B.Cu") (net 12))
 (segment (start 145.9533 79.484) (end 145.9533 78.4323) (width 0.2) (layer "F.Cu") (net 10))
 (segment (start 181.4296 78.4323) (end 181.6129 78.6156) (width 0.2) (layer "F.Cu") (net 10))
 (segment (start 145.9533 78.4323) (end 181.4296 78.4323) (width 0.2) (layer "F.Cu") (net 10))
 (via (at 181.6129 78.6156) (size 0.6) (drill 0.3) (layers "F.Cu" "B.Cu") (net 10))
 (segment (start 184.7635 110.3529) (end 184.9283 110.5177) (width 0.2) (layer "B.Cu") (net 10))
 (segment (start 184.9283 110.5177) (end 184.9283 113.9283) (width 0.2) (layer "B.Cu") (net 10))
 (segment (start 184.7635 110.3529) (end 184.9283 110.5177) (width 0.2) (layer "B.Cu") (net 10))
 (segment (start 184.5281 110.1175) (end 184.7635 110.3529) (width 0.2) (layer "B.Cu") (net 10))
 (segment (start 181.6129 78.6156) (end 184.5281 81.5308) (width 0.2) (layer "B.Cu") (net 10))
 (segment (start 184.5281 81.5308) (end 184.5281 110.1175) (width 0.2) (layer "B.Cu") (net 10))
 (segment (start 184.9283 113.9283) (end 186 115) (width 0.2) (layer "B.Cu") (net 10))
 (segment (start 184.0567 117.1464) (end 173.2196 117.1464) (width 0.2) (layer "F.Cu") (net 6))
 (segment (start 171.4803 117.584) (end 172.782 117.584) (width 0.2) (layer "F.Cu") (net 6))
 (segment (start 173.2196 117.1464) (end 172.782 117.584) (width 0.2) (layer "F.Cu") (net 6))
 (via (at 184.0567 117.1464) (size 0.6) (drill 0.3) (layers "F.Cu" "B.Cu") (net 6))
 (segment (start 186.9574 115.3749) (end 185.1859 117.1464) (width 0.2) (layer "B.Cu") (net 6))
 (segment (start 186.9574 111.7786) (end 186.9574 115.3749) (width 0.2) (layer "B.Cu") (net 6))
 (segment (start 185.1859 117.1464) (end 184.0567 117.1464) (width 0.2) (layer "B.Cu") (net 6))
 (segment (start 185.0711 109.8923) (end 186.9574 111.7786) (width 0.2) (layer "B.Cu") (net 6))
 (segment (start 185.0711 80.4361) (end 185.0711 109.8923) (width 0.2) (layer "B.Cu") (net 6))
 (segment (start 184.595 79.96) (end 185.0711 80.4361) (width 0.2) (layer "B.Cu") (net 6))
 (segment (start 168.8458 118.1415) (end 170.7368 116.2505) (width 0.2) (layer "F.Cu") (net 14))
 (segment (start 176 115) (end 175.0733 115) (width 0.2) (layer "F.Cu") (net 14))
 (segment (start 173.8228 116.2505) (end 175.0733 115) (width 0.2) (layer "F.Cu") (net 14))
 (segment (start 149.1211 118.1415) (end 168.8458 118.1415) (width 0.2) (layer "F.Cu") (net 14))
 (segment (start 170.7368 116.2505) (end 173.8228 116.2505) (width 0.2) (layer "F.Cu") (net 14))
 (via (at 149.1211 118.1415) (size 0.6) (drill 0.3) (layers "F.Cu" "B.Cu") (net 14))
 (segment (start 146.3477 90.6957) (end 149.1211 93.4691) (width 0.2) (layer "B.Cu") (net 14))
 (segment (start 145.9533 89.644) (end 145.9533 90.6957) (width 0.2) (layer "B.Cu") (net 14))
 (segment (start 149.1211 93.4691) (end 149.1211 118.1415) (width 0.2) (layer "B.Cu") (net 14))
 (segment (start 145.9533 90.6957) (end 146.3477 90.6957) (width 0.2) (layer "B.Cu") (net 14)))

